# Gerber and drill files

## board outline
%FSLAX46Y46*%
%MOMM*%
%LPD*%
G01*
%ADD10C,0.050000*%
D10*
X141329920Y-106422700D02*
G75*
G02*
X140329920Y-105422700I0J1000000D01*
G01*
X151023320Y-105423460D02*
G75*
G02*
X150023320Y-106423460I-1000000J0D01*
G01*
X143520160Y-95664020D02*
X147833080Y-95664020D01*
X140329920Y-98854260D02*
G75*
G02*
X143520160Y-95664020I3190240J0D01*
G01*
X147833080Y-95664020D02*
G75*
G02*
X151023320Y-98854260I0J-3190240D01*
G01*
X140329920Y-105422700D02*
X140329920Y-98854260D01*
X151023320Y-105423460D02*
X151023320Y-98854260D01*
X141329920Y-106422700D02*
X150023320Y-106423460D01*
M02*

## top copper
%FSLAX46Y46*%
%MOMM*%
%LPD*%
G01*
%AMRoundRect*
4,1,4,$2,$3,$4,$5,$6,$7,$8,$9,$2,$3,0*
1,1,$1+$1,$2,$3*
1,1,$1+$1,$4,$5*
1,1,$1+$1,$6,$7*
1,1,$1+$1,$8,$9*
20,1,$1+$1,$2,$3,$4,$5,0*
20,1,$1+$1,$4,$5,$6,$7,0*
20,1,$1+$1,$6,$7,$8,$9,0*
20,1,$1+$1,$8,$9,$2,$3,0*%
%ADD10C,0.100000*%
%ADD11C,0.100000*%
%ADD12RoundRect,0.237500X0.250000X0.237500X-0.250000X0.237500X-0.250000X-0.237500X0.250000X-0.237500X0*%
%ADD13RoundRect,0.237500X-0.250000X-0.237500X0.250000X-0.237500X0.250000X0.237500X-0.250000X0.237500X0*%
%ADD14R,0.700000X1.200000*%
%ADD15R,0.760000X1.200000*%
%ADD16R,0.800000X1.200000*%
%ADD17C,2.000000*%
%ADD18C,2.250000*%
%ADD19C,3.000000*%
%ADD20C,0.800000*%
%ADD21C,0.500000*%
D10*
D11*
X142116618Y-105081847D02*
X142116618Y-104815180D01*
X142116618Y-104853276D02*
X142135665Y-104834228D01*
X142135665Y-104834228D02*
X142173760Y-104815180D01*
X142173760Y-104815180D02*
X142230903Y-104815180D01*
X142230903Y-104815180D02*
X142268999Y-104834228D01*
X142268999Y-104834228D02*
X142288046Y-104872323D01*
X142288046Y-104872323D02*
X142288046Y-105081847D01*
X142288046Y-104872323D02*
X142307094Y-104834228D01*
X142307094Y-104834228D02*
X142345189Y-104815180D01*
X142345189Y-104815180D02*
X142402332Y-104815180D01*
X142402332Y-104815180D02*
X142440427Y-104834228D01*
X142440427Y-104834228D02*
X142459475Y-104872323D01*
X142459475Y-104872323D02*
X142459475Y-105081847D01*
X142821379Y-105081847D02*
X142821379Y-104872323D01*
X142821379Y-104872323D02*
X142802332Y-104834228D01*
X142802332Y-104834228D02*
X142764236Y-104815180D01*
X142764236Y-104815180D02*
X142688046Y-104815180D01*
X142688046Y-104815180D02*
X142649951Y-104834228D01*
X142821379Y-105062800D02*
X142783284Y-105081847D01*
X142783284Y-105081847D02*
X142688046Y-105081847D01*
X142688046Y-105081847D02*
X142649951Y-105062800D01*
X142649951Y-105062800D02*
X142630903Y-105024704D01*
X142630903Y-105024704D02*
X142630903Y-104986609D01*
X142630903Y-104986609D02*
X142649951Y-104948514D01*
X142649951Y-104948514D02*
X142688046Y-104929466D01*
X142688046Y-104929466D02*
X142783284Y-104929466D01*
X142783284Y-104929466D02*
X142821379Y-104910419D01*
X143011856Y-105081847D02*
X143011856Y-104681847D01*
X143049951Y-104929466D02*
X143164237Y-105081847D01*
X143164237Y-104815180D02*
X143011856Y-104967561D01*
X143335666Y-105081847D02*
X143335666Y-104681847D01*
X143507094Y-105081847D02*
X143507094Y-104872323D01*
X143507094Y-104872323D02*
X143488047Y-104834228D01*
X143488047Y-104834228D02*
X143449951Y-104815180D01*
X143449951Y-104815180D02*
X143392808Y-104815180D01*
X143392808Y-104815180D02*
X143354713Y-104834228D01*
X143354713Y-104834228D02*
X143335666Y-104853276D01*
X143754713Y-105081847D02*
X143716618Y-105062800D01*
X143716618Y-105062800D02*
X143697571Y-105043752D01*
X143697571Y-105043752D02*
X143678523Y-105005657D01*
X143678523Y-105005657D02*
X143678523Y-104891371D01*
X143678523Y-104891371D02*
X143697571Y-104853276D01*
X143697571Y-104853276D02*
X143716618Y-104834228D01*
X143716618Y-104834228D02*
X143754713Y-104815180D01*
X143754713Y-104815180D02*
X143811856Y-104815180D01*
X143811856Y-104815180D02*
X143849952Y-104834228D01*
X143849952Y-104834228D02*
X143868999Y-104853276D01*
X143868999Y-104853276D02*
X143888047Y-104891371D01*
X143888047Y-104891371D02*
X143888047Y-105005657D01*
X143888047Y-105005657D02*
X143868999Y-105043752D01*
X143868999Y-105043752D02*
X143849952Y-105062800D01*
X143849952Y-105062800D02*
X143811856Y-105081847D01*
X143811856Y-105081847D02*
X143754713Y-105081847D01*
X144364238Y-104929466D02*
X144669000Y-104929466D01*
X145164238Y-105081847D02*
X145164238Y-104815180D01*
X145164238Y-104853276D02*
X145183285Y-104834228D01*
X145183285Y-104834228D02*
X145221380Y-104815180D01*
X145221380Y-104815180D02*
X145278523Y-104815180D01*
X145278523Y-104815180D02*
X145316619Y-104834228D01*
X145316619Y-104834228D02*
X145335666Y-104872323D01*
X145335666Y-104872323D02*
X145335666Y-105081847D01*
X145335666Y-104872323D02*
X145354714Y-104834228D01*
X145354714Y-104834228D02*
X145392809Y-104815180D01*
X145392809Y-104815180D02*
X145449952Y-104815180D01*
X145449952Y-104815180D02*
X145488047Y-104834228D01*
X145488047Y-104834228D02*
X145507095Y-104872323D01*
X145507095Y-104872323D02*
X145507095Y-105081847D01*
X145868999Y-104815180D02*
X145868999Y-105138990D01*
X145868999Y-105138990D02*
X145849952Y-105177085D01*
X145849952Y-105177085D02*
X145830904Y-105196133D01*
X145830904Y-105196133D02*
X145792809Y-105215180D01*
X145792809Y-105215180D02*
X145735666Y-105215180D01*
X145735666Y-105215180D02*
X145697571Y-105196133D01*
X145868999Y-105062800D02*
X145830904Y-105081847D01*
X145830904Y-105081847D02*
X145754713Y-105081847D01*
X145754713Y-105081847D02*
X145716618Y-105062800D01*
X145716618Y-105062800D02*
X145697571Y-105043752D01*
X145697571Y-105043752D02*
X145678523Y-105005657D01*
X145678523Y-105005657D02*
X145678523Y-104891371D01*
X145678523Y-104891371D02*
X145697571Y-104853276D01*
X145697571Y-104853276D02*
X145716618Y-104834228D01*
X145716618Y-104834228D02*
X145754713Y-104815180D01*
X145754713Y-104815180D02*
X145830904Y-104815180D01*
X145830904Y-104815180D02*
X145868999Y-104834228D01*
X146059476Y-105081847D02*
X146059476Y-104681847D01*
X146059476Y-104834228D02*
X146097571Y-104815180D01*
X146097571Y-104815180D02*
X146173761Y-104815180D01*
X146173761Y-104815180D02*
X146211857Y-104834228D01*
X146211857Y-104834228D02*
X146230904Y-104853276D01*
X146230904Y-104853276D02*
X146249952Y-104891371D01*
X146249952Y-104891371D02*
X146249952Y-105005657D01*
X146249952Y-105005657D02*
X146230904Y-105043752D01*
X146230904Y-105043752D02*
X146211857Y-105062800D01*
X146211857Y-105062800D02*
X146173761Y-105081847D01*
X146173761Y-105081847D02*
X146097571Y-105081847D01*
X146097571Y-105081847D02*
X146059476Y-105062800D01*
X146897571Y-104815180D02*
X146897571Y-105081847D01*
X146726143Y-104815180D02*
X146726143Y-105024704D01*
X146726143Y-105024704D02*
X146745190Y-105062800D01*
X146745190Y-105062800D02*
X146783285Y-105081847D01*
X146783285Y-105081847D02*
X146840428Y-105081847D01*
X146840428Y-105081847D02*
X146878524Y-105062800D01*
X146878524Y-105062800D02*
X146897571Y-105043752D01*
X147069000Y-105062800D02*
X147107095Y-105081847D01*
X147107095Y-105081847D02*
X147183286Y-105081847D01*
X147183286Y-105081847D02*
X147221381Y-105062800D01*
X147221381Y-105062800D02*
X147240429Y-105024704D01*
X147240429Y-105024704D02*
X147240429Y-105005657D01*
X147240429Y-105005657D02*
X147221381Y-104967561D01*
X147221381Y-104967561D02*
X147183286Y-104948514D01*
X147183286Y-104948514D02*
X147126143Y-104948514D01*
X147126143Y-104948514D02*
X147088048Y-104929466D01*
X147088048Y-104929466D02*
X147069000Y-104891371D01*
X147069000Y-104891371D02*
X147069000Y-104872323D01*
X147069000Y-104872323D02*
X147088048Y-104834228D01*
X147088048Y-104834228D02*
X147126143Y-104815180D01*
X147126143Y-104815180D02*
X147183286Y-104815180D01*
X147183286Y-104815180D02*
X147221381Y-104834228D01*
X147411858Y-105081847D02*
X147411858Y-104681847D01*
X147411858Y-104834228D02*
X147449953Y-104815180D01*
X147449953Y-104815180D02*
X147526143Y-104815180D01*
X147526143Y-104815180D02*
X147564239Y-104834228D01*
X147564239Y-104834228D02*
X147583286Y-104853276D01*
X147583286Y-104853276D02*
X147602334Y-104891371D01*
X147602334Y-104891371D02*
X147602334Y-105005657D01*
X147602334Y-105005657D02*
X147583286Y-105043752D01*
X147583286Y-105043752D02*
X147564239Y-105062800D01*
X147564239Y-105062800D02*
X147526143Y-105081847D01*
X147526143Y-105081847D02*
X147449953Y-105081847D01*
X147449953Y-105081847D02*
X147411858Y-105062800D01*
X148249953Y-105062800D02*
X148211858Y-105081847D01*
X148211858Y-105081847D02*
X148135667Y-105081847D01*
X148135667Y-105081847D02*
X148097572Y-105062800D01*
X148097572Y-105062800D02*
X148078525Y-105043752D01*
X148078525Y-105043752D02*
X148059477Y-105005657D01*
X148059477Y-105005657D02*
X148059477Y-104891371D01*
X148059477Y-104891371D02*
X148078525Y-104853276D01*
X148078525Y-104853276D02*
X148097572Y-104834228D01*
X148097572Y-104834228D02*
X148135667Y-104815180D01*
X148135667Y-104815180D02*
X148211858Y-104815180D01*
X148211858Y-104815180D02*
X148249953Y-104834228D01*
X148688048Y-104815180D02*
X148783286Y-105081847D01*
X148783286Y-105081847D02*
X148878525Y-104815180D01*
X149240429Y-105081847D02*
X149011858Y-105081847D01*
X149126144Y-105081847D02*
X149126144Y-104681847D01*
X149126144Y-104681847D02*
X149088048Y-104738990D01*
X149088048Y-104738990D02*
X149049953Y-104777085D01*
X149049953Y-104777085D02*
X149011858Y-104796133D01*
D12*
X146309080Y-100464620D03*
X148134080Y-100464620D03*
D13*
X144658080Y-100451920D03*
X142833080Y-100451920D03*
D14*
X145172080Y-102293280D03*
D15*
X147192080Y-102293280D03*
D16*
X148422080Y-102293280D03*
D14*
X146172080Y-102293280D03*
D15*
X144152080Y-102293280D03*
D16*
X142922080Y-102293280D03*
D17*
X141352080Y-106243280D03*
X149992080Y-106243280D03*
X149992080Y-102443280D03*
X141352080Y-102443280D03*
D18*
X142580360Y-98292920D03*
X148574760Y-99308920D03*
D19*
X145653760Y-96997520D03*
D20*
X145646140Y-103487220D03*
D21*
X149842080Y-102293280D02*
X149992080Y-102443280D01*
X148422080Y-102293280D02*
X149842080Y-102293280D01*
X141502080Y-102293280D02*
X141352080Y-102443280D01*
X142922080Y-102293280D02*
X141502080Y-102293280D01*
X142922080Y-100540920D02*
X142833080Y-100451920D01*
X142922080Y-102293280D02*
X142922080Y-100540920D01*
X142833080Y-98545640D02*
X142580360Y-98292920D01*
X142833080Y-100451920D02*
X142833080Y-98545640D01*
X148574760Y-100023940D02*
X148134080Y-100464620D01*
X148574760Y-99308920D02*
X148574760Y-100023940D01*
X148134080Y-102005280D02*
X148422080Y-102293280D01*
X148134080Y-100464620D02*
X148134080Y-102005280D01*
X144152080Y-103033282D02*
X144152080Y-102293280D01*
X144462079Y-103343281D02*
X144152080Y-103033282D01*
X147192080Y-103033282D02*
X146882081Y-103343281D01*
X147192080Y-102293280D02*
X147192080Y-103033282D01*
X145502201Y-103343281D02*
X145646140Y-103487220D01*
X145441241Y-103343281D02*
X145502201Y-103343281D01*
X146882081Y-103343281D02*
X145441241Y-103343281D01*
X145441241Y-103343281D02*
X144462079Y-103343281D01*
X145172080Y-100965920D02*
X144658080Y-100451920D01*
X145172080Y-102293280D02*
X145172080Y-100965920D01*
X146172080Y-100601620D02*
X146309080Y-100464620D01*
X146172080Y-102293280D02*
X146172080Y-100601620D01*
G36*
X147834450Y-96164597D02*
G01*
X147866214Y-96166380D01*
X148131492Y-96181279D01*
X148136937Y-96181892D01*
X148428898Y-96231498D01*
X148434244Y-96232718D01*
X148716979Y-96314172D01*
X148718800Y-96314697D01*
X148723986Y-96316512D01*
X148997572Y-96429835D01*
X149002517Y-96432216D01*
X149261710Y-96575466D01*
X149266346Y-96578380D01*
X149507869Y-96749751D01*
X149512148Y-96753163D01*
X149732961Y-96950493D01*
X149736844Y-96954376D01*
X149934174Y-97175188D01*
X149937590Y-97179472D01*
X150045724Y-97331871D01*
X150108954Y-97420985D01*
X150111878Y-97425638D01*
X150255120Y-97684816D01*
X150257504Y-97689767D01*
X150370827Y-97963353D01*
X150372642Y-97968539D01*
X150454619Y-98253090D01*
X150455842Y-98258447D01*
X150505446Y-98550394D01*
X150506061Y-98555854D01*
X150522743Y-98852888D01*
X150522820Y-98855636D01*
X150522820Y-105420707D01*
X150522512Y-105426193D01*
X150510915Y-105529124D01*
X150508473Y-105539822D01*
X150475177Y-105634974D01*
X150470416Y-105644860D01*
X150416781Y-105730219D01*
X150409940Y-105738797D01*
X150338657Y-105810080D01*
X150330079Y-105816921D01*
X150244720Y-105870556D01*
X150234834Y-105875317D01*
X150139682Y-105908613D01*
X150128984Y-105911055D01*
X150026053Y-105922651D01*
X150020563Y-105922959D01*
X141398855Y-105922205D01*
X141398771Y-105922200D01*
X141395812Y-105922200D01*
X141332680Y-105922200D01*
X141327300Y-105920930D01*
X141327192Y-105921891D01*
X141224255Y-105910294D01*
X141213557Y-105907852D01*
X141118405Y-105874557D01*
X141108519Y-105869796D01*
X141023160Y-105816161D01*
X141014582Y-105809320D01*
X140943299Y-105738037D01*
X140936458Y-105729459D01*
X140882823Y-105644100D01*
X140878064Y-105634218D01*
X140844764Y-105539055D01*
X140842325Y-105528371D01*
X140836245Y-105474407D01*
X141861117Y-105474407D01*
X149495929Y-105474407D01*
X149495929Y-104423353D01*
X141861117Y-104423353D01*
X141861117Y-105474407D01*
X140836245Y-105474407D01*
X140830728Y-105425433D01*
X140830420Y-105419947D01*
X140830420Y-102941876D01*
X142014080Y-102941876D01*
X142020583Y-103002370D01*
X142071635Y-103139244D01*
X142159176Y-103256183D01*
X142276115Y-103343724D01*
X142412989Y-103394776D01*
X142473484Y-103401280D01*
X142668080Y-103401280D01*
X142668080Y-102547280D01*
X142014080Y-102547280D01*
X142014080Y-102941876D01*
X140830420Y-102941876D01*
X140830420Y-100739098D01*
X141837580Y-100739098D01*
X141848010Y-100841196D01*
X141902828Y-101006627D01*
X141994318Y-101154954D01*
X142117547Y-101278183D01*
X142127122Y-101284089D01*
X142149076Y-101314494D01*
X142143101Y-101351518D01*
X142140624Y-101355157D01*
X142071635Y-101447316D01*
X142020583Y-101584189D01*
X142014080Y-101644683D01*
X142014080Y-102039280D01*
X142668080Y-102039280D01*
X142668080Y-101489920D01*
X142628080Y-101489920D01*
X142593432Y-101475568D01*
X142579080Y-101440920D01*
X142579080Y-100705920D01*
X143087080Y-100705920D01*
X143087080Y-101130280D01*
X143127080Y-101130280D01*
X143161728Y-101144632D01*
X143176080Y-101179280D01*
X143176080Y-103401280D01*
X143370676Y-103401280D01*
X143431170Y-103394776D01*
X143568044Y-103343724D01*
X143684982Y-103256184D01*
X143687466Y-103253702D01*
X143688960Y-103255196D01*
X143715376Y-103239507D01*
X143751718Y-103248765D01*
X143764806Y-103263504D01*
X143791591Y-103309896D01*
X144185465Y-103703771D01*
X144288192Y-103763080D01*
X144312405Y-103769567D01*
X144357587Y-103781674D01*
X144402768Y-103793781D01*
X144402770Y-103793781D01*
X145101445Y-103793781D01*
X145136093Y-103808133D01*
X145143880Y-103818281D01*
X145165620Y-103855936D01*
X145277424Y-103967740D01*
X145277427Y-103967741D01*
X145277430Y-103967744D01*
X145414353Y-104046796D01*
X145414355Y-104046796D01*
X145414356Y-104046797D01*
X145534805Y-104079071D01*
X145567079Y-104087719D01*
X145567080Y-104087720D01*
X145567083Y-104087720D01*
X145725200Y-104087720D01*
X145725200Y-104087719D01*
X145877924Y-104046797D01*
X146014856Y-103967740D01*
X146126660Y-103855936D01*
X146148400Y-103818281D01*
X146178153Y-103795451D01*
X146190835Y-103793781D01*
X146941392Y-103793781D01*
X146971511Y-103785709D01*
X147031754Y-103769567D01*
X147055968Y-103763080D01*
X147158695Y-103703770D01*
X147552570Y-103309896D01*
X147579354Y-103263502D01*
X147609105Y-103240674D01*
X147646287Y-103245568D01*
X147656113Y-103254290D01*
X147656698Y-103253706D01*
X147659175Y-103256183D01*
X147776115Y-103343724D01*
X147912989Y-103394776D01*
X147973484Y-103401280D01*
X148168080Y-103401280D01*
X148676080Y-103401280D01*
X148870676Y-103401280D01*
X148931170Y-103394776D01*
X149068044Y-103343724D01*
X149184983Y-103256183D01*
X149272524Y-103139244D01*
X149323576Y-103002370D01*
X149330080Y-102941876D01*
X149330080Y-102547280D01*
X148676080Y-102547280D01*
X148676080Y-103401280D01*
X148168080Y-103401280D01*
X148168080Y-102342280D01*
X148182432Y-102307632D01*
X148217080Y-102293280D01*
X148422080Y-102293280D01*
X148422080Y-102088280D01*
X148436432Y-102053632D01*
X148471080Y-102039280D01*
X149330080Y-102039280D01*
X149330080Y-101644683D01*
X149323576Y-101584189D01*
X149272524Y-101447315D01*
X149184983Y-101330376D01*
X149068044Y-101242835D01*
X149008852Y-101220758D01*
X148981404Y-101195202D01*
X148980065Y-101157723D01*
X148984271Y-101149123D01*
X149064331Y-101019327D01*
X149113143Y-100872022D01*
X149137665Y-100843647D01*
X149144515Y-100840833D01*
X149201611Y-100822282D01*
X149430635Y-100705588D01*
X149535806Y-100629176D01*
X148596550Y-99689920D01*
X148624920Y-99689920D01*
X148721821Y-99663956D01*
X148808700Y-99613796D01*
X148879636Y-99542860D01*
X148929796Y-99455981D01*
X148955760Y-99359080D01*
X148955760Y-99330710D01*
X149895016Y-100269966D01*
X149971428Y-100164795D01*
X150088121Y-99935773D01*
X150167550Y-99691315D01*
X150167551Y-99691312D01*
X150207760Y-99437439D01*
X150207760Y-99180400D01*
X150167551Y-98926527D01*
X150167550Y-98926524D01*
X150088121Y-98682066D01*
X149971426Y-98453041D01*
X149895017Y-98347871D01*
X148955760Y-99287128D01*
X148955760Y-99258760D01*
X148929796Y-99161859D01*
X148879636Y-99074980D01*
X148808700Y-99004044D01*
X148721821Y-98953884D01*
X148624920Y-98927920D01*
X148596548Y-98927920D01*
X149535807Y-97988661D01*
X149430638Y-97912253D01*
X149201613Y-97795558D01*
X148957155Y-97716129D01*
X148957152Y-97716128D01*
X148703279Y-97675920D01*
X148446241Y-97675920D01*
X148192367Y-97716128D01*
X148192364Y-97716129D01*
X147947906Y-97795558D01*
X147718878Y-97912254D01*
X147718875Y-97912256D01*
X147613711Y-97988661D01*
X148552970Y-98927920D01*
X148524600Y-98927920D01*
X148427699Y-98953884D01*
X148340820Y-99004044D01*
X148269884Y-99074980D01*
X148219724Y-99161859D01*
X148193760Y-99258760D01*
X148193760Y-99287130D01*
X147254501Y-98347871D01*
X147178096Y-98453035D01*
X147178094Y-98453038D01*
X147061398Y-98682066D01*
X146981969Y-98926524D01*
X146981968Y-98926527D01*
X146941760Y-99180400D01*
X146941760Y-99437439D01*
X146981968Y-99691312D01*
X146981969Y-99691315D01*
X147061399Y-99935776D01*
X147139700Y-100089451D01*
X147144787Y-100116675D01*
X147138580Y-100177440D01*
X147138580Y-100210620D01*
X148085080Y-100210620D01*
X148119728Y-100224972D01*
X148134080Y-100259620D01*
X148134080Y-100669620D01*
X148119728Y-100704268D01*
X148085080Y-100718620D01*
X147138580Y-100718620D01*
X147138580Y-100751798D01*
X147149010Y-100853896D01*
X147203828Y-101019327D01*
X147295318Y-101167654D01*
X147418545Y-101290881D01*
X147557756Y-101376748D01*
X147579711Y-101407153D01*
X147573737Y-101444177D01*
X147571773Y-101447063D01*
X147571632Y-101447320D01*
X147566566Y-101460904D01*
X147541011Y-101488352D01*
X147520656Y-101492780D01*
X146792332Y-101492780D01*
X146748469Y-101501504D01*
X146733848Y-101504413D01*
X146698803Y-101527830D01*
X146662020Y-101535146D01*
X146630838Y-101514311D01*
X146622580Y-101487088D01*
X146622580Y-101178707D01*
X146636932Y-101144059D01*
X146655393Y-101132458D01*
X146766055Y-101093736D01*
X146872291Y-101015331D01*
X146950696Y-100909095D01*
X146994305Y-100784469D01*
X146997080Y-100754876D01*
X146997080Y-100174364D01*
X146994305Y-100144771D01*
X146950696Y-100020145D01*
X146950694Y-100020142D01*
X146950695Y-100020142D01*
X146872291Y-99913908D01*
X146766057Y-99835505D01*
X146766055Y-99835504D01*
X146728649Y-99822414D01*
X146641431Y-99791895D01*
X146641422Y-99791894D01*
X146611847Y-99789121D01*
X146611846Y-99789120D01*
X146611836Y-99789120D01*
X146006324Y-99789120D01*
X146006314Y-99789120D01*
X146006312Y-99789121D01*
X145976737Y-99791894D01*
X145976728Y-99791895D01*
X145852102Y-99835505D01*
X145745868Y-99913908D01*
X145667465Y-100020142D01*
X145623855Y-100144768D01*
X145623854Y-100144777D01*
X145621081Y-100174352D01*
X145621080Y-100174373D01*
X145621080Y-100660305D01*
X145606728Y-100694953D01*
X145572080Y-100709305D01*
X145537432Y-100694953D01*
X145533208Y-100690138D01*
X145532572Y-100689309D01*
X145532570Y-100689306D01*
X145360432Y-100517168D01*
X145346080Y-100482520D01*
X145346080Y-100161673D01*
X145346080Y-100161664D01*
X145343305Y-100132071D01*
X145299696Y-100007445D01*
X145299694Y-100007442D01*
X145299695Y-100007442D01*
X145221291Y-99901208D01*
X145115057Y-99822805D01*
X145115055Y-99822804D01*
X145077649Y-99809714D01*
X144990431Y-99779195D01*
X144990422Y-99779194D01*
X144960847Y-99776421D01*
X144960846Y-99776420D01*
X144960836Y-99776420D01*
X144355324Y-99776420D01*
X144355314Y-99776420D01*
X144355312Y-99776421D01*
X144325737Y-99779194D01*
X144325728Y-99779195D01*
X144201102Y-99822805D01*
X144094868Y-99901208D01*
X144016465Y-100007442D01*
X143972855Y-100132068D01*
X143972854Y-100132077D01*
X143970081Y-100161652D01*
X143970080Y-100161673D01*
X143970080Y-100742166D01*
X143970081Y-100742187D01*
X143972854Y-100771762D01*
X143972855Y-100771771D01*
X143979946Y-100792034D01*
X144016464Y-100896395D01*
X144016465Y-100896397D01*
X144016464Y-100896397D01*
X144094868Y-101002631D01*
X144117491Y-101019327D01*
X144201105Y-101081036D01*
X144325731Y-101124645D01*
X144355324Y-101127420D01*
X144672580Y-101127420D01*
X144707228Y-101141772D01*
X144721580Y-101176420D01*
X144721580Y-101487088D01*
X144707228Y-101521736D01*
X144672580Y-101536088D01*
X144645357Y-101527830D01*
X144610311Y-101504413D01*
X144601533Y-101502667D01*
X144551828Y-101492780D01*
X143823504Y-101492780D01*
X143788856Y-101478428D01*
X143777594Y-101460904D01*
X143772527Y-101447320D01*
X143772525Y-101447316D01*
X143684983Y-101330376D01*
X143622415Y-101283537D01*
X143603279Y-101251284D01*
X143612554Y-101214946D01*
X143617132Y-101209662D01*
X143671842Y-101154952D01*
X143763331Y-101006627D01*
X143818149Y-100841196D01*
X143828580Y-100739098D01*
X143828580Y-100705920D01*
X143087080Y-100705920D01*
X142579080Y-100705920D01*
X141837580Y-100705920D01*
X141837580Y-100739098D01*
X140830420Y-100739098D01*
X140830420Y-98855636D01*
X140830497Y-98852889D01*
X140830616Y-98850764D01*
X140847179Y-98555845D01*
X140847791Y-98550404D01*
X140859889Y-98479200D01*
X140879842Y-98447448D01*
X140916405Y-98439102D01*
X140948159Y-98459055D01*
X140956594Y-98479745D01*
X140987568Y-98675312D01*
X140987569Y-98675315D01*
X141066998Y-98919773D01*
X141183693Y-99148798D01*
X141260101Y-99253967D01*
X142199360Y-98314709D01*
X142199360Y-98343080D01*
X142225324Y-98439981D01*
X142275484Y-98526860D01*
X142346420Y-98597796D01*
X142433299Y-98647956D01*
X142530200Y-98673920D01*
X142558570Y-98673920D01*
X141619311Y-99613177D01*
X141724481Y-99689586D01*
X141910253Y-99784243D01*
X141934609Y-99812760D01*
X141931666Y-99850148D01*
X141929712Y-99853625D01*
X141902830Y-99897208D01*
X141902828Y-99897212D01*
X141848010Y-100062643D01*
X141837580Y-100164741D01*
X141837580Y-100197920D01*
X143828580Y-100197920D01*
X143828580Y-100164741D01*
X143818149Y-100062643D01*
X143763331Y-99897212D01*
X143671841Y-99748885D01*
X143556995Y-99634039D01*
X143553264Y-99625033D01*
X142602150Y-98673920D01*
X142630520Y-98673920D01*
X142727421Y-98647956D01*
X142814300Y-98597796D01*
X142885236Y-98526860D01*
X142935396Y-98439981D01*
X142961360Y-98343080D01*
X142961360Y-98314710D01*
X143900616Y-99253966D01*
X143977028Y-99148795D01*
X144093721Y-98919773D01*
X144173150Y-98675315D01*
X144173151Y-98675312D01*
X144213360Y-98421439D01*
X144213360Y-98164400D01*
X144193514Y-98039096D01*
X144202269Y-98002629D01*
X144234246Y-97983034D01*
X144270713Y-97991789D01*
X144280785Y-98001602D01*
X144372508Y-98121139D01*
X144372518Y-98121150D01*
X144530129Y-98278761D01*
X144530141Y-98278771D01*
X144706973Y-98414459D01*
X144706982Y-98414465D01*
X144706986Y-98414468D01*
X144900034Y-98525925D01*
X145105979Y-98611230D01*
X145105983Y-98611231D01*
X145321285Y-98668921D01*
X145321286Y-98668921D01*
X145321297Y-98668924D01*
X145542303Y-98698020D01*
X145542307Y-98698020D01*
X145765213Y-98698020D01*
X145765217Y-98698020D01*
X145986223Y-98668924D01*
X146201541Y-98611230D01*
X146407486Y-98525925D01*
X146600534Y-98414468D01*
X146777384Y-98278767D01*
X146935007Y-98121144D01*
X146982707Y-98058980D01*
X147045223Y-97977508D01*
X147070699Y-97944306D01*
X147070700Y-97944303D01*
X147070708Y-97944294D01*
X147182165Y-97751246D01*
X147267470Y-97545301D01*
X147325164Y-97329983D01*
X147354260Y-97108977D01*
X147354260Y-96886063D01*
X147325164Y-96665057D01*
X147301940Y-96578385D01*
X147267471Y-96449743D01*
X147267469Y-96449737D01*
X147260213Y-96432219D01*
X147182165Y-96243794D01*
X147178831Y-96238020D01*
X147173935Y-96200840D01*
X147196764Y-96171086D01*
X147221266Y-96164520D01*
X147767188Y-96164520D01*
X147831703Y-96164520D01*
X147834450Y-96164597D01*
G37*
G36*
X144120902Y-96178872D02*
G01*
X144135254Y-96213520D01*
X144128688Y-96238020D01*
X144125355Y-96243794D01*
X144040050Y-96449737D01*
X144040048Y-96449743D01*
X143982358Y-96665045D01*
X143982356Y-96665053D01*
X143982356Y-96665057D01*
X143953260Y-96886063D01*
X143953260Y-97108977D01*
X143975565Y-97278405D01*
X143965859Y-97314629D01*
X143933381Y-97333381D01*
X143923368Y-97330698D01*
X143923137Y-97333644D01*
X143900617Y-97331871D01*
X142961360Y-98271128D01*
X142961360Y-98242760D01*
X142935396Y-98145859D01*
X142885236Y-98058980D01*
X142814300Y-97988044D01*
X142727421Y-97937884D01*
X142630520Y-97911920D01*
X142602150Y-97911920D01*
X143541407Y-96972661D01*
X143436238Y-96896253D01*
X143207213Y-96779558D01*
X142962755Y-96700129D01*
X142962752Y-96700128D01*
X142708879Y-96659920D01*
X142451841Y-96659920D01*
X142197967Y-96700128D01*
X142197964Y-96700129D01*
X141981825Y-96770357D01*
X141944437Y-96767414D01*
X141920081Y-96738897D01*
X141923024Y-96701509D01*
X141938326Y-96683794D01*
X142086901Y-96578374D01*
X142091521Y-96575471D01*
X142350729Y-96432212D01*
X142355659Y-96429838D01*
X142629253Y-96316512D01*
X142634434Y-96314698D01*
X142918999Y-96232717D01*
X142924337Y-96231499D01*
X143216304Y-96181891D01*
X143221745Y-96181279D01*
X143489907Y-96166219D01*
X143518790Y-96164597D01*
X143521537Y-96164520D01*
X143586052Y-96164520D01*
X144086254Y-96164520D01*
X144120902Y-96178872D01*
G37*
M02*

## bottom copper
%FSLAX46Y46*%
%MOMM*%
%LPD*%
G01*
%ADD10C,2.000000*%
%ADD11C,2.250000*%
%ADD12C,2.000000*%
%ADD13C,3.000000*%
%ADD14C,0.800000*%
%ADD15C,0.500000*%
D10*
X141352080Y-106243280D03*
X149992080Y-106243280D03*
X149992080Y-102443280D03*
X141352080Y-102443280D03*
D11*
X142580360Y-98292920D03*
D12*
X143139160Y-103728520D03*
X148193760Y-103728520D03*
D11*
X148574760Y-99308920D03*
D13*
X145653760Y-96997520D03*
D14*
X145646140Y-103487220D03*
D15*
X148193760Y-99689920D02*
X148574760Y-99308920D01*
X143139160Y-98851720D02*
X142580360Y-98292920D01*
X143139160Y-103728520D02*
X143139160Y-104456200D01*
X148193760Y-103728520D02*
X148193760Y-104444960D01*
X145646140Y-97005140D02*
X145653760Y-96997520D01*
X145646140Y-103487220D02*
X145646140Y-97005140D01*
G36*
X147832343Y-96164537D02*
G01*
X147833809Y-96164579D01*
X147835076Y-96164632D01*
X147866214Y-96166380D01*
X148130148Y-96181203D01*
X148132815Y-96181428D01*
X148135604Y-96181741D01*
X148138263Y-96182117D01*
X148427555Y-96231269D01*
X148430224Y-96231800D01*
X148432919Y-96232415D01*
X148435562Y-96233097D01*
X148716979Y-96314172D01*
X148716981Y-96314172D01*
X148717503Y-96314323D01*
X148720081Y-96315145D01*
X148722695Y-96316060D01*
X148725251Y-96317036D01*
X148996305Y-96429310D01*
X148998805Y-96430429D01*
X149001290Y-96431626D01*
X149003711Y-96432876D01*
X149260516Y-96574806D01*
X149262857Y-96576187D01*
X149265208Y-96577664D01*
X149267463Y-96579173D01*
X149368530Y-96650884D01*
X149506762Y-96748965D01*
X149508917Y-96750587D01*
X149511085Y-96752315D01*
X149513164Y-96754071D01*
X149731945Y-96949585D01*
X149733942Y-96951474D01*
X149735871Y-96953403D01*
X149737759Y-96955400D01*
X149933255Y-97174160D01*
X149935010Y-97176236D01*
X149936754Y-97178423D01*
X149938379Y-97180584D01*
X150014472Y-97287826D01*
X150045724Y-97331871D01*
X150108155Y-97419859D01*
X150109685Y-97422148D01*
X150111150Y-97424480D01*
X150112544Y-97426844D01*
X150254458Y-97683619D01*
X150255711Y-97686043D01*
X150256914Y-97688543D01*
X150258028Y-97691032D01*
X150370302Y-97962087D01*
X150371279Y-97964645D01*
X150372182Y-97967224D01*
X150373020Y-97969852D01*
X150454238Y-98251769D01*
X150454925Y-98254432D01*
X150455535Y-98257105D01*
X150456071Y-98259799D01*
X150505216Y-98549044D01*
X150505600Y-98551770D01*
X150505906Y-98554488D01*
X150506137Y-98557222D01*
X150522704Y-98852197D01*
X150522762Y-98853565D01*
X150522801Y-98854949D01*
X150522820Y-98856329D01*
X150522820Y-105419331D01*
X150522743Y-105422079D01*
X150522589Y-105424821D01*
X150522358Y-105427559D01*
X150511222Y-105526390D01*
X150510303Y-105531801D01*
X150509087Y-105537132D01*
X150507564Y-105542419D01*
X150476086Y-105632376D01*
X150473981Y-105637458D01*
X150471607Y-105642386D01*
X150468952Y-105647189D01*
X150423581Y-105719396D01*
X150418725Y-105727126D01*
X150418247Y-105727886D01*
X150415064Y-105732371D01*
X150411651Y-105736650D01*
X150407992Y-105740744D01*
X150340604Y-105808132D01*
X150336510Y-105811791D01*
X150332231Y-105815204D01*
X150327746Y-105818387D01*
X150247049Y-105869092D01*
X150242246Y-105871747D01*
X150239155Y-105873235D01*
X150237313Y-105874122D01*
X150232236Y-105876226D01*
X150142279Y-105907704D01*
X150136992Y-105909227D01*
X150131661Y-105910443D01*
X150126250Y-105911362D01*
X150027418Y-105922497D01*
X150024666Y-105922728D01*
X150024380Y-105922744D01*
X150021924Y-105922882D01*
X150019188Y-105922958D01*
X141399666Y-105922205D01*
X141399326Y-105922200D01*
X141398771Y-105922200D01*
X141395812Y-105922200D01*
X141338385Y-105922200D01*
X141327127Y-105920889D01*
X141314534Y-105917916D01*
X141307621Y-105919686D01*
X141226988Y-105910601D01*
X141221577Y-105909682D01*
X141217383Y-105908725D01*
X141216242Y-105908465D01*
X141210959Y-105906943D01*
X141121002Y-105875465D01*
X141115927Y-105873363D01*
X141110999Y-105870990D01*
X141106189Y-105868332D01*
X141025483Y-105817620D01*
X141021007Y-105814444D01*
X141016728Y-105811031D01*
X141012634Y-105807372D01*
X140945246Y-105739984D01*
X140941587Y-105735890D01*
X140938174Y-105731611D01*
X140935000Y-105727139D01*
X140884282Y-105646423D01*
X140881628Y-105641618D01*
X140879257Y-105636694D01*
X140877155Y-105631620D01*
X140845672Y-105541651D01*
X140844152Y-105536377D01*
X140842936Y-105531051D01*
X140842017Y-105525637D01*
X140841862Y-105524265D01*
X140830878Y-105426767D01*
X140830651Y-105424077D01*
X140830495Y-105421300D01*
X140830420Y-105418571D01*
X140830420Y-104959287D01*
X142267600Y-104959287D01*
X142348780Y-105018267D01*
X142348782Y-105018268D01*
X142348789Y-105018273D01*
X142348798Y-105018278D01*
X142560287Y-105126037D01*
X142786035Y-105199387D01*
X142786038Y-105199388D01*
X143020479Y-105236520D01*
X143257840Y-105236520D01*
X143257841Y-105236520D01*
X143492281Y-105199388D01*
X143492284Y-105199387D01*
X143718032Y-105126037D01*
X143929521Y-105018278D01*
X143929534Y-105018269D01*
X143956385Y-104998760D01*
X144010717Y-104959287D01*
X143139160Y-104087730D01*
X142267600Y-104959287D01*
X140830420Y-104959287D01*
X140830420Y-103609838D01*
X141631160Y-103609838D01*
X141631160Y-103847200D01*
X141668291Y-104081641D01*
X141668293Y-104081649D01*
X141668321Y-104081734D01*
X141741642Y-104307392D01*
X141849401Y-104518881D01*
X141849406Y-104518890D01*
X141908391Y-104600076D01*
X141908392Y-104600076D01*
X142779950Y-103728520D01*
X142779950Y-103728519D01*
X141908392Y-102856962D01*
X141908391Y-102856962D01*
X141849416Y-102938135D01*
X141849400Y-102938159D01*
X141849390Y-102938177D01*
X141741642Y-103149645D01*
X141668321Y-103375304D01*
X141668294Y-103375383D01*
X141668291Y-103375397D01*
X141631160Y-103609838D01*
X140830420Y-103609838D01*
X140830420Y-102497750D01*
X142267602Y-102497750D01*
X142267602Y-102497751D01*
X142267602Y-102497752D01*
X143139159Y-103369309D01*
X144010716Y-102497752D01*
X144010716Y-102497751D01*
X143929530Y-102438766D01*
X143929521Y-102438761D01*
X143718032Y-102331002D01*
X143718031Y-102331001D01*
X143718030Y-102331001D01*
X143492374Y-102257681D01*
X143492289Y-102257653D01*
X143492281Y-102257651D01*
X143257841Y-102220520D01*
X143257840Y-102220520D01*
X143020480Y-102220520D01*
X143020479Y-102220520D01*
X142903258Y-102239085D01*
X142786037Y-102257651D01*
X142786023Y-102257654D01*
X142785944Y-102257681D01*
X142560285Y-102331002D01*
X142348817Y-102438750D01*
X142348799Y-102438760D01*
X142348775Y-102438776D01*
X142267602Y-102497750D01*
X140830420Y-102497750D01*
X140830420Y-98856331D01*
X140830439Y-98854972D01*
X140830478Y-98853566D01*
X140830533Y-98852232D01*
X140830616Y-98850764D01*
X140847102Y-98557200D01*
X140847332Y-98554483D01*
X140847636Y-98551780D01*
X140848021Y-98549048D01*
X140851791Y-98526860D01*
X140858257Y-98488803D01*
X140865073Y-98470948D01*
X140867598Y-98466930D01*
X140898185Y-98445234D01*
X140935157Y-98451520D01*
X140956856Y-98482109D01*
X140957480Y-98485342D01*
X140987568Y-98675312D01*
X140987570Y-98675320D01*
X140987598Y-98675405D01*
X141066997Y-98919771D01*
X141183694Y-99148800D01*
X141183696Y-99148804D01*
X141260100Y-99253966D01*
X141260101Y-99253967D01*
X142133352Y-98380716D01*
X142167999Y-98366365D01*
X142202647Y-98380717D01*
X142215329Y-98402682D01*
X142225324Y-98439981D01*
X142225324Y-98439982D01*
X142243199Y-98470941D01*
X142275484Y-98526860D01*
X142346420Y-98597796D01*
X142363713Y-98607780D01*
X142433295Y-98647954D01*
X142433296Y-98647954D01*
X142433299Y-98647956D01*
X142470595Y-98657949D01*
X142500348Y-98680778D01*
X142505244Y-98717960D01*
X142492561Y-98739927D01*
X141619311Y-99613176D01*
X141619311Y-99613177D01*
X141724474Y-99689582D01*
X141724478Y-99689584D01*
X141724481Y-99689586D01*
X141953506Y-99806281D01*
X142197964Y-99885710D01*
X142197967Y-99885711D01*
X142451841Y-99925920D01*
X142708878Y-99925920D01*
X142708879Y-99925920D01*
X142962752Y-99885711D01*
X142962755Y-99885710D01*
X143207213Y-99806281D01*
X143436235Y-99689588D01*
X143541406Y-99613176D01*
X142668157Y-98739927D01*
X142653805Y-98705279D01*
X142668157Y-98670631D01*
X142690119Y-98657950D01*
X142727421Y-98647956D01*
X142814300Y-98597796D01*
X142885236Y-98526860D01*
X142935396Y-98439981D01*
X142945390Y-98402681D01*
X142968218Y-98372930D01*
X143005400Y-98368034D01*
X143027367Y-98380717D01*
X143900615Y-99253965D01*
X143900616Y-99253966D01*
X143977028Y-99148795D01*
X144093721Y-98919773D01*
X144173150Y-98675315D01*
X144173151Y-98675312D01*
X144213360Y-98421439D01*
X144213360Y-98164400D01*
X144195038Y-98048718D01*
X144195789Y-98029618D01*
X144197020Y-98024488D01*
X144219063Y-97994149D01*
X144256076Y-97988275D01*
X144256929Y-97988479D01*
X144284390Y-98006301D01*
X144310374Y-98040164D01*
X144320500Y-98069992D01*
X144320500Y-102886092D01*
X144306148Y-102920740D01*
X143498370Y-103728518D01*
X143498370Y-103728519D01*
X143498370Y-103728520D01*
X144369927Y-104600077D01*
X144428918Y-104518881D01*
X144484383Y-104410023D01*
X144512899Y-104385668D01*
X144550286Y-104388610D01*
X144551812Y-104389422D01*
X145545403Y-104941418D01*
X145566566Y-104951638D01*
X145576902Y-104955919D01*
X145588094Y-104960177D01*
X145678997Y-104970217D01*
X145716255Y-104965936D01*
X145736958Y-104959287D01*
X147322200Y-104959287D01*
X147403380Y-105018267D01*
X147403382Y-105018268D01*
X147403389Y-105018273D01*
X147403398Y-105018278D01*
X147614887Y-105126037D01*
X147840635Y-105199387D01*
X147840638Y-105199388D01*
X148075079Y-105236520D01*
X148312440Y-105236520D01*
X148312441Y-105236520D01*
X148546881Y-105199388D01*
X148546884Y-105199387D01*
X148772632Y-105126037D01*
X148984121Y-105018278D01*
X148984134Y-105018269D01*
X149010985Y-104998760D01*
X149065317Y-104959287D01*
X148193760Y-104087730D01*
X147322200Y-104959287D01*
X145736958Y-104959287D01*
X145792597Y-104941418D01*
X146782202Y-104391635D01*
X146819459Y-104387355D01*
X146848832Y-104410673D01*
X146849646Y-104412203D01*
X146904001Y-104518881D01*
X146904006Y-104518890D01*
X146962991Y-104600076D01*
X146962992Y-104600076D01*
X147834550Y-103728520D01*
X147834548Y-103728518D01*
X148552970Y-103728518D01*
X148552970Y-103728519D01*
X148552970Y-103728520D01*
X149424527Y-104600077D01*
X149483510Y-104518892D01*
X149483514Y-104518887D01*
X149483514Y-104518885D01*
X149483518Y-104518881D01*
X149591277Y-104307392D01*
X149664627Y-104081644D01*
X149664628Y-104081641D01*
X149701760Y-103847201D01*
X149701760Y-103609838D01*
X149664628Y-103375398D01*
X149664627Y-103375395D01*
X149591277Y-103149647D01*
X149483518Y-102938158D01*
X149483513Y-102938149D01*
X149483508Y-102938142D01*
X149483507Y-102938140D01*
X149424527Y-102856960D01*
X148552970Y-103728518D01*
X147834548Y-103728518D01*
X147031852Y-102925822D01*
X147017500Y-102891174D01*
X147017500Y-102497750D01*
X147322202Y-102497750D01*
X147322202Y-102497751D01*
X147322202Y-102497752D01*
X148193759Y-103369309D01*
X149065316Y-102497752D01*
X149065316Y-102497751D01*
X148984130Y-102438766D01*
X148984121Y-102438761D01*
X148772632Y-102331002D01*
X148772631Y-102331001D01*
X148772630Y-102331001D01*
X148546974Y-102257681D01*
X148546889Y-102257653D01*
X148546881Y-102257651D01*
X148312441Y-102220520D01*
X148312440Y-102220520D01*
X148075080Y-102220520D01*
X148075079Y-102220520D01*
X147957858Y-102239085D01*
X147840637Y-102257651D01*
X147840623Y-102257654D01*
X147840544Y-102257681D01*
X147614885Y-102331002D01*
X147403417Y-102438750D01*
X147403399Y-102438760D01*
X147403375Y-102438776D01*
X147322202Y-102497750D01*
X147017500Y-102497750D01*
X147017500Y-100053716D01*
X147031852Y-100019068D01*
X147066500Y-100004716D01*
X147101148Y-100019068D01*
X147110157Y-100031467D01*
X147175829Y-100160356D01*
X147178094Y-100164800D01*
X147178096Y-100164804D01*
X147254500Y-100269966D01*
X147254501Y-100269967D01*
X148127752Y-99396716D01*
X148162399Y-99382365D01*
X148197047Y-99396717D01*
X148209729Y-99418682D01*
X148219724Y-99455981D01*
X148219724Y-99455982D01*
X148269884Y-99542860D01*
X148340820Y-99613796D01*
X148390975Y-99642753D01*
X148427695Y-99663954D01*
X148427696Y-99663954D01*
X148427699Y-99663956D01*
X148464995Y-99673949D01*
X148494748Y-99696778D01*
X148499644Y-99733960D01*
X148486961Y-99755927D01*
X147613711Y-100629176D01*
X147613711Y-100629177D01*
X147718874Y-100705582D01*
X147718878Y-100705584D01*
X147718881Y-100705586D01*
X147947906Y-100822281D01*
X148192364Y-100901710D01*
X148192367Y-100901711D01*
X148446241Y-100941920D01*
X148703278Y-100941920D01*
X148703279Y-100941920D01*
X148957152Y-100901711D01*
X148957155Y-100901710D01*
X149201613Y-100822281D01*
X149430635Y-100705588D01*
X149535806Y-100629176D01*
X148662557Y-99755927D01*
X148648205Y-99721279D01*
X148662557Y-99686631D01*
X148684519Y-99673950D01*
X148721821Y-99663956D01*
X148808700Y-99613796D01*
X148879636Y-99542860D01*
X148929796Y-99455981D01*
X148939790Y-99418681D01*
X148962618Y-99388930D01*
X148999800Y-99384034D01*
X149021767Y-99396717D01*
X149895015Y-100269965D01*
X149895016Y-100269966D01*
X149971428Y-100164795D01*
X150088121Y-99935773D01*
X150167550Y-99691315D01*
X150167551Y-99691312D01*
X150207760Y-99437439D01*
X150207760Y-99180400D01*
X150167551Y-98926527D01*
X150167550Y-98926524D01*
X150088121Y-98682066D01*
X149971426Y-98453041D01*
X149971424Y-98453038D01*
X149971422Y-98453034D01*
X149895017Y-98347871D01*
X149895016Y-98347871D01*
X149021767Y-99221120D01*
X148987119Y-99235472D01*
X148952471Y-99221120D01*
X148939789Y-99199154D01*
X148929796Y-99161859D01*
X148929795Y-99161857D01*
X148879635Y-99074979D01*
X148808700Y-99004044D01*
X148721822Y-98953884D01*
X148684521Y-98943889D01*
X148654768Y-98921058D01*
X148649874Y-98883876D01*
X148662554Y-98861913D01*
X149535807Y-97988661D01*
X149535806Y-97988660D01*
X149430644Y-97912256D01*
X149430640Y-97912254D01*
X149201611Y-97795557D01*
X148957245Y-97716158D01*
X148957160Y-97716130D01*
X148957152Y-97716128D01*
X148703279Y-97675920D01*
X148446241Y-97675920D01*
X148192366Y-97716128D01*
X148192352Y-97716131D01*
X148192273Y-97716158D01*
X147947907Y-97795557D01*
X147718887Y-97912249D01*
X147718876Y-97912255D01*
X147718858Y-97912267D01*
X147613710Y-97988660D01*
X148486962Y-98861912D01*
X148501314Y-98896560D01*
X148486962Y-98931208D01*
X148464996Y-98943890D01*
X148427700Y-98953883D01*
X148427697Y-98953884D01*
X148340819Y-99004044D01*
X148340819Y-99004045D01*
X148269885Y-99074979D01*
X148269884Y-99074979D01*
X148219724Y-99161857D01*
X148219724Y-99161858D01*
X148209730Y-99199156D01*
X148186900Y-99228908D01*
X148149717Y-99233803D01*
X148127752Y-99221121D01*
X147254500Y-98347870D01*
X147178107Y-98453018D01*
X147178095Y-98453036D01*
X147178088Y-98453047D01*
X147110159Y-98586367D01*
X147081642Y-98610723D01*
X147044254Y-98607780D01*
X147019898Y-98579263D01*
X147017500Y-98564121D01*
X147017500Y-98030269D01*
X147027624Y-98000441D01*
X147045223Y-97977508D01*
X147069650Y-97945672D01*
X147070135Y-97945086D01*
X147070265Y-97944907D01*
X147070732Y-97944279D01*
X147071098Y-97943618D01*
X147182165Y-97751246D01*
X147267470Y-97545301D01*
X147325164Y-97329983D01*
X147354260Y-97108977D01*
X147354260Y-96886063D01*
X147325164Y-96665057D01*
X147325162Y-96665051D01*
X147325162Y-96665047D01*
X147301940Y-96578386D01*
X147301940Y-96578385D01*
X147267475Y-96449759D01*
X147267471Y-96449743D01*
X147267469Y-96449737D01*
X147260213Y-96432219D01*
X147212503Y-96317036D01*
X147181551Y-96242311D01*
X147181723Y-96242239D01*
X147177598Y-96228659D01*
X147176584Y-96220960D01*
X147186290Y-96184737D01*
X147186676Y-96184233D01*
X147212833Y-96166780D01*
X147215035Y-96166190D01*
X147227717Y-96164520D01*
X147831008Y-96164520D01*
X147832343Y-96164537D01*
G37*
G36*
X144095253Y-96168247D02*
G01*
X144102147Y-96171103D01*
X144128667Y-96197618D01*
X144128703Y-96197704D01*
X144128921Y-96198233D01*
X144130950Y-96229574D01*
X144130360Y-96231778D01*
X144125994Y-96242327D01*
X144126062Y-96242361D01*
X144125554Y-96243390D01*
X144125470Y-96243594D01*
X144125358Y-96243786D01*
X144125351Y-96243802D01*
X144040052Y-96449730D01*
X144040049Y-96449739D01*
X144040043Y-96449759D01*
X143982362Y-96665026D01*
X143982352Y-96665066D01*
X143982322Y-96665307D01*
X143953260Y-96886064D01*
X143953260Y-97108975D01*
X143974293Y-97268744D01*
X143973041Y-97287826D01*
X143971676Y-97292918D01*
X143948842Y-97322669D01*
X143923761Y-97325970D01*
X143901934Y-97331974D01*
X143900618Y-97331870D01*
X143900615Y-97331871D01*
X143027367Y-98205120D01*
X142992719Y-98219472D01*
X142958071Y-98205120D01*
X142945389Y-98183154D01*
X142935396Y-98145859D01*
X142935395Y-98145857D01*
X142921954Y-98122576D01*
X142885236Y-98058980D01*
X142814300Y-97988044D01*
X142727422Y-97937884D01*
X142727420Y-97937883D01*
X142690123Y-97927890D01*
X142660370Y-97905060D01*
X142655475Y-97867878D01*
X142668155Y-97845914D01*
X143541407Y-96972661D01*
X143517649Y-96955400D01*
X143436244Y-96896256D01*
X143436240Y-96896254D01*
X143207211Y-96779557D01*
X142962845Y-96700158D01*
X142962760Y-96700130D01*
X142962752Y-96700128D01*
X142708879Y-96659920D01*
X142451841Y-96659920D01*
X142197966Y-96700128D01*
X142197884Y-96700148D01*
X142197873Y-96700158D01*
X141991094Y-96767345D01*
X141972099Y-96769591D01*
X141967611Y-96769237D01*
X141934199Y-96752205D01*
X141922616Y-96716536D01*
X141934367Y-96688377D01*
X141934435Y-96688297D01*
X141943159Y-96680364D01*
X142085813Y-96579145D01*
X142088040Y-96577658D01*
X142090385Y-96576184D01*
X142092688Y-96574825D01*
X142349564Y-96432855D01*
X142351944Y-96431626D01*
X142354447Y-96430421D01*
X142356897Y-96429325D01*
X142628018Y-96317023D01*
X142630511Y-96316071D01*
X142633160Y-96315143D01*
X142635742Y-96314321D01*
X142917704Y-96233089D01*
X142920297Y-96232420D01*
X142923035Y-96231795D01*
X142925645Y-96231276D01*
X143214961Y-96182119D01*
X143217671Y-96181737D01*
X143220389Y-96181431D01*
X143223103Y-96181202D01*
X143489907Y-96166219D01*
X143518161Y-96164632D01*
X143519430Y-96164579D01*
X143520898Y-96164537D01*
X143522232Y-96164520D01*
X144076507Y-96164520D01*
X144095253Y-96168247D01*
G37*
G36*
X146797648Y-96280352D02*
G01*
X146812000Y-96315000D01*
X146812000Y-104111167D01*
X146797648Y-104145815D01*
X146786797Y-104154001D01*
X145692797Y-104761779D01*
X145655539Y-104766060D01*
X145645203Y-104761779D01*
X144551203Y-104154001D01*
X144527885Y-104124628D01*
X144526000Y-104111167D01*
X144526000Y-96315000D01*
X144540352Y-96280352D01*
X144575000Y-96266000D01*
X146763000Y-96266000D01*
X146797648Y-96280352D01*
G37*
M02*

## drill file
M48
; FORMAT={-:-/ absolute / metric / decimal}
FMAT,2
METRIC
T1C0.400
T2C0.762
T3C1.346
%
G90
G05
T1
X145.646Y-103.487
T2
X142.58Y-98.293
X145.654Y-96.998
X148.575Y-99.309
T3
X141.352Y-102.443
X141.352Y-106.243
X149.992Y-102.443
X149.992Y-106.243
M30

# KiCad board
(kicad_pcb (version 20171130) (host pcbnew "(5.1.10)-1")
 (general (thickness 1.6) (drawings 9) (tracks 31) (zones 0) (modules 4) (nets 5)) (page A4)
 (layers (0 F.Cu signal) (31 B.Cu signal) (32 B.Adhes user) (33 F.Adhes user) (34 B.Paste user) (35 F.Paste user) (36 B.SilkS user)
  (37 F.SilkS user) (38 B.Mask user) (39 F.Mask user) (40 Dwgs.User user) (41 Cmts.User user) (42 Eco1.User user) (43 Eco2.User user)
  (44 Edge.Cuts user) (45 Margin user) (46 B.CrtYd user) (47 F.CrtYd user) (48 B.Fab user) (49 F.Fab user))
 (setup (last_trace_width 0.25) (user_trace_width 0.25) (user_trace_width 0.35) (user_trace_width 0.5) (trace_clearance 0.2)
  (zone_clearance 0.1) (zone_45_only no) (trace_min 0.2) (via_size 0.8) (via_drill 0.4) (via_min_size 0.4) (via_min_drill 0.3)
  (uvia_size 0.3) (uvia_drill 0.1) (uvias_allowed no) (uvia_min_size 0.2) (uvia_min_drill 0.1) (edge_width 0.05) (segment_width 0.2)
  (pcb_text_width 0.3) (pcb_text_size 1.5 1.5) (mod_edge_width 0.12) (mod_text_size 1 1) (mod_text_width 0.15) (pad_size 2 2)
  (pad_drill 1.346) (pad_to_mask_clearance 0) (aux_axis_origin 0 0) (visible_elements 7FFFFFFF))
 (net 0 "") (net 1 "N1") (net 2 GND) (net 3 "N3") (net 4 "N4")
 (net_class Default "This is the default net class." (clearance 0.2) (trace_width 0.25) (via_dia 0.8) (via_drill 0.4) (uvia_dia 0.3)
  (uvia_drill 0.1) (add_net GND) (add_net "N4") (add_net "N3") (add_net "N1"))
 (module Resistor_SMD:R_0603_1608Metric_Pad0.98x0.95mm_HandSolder (layer F.Cu) (at 147.22158 100.46462 180)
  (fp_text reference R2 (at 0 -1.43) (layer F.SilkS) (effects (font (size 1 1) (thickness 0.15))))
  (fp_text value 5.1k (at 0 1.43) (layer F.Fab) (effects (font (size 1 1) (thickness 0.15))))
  (pad 2 smd roundrect (at 0.9125 0 180) (size 0.975 0.95) (layers F.Cu F.Paste F.Mask) (roundrect_rratio 0.25) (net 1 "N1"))
  (pad 1 smd roundrect (at -0.9125 0 180) (size 0.975 0.95) (layers F.Cu F.Paste F.Mask) (roundrect_rratio 0.25) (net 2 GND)))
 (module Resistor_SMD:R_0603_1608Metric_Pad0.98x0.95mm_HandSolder (layer F.Cu) (at 143.74558 100.45192)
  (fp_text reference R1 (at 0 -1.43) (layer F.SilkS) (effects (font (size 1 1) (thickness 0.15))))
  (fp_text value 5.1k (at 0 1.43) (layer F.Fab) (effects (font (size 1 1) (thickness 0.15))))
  (pad 2 smd roundrect (at 0.9125 0) (size 0.975 0.95) (layers F.Cu F.Paste F.Mask) (roundrect_rratio 0.25) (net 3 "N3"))
  (pad 1 smd roundrect (at -0.9125 0) (size 0.975 0.95) (layers F.Cu F.Paste F.Mask) (roundrect_rratio 0.25) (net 2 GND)))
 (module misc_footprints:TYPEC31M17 (layer F.Cu) (at 145.67208 104.79328)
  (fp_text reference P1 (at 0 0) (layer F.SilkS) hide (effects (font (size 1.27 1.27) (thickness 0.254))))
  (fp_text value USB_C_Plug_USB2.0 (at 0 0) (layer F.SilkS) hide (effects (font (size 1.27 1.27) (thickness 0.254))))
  (pad A5 smd rect (at -0.5 -2.5) (size 0.7 1.2) (layers F.Cu F.Paste F.Mask) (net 3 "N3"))
  (pad A9 smd rect (at 1.52 -2.5) (size 0.76 1.2) (layers F.Cu F.Paste F.Mask) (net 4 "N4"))
  (pad A12 smd rect (at 2.75 -2.5) (size 0.8 1.2) (layers F.Cu F.Paste F.Mask) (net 2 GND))
  (pad B5 smd rect (at 0.5 -2.5) (size 0.7 1.2) (layers F.Cu F.Paste F.Mask) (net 1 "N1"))
  (pad B9 smd rect (at -1.52 -2.5) (size 0.76 1.2) (layers F.Cu F.Paste F.Mask) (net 4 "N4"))
  (pad B12 smd rect (at -2.75 -2.5) (size 0.8 1.2) (layers F.Cu F.Paste F.Mask) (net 2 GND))
  (pad MH1 thru_hole circle (at -4.32 1.45) (size 2 2) (drill 1.346) (layers *.Cu *.Mask) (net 2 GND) (zone_connect 2))
  (pad MH2 thru_hole circle (at 4.32 1.45) (size 2 2) (drill 1.346) (layers *.Cu *.Mask) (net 2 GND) (zone_connect 2))
  (pad MH3 thru_hole circle (at 4.32 -2.35) (size 2 2) (drill 1.346) (layers *.Cu *.Mask) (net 2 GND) (zone_connect 2))
  (pad MH4 thru_hole circle (at -4.32 -2.35) (size 2 2) (drill 1.346) (layers *.Cu *.Mask) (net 2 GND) (zone_connect 2)))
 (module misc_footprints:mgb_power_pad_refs (layer F.Cu) (at 150.12416 101.29012)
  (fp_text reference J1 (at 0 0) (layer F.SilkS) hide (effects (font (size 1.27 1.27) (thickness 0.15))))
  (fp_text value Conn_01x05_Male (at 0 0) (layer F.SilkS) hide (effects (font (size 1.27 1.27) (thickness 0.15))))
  (pad 2 thru_hole circle (at -7.5438 -2.9972) (size 2.25 2.25) (drill 0.762) (layers *.Cu *.Mask) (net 2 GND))
  (pad 4 smd circle (at -6.985 2.4384) (size 2 2) (layers B.Cu B.Paste B.Mask) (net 2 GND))
  (pad 5 smd circle (at -1.9304 2.4384) (size 2 2) (layers B.Cu B.Paste B.Mask) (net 2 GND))
  (pad 3 thru_hole circle (at -1.5494 -1.9812) (size 2.25 2.25) (drill 0.762) (layers *.Cu *.Mask) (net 2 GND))
  (pad 1 thru_hole circle (at -4.4704 -4.2926) (size 3 3) (drill 0.762) (layers *.Cu *.Mask) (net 4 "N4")))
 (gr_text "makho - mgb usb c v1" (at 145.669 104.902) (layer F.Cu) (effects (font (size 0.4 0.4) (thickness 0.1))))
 (gr_arc (start 141.32992 105.4227) (end 140.32992 105.4227) (angle -90) (layer Edge.Cuts) (width 0.05))
 (gr_arc (start 150.02332 105.42346) (end 150.02332 106.42346) (angle -90) (layer Edge.Cuts) (width 0.05))
 (gr_line (start 143.52016 95.66402) (end 147.83308 95.66402) (layer Edge.Cuts) (width 0.05))
 (gr_arc (start 143.52016 98.85426) (end 143.52016 95.66402) (angle -90) (layer Edge.Cuts) (width 0.05))
 (gr_arc (start 147.83308 98.85426) (end 151.02332 98.85426) (angle -90) (layer Edge.Cuts) (width 0.05))
 (gr_line (start 140.32992 105.4227) (end 140.32992 98.85426) (layer Edge.Cuts) (width 0.05))
 (gr_line (start 151.02332 105.42346) (end 151.02332 98.85426) (layer Edge.Cuts) (width 0.05))
 (gr_line (start 141.32992 106.4227) (end 150.02332 106.42346) (layer Edge.Cuts) (width 0.05))
 (segment (start 149.84208 102.29328) (end 149.99208 102.44328) (width 0.5) (layer F.Cu) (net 2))
 (segment (start 148.42208 102.29328) (end 149.84208 102.29328) (width 0.5) (layer F.Cu) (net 2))
 (segment (start 141.50208 102.29328) (end 141.35208 102.44328) (width 0.5) (layer F.Cu) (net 2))
 (segment (start 142.92208 102.29328) (end 141.50208 102.29328) (width 0.5) (layer F.Cu) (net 2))
 (segment (start 142.92208 100.54092) (end 142.83308 100.45192) (width 0.5) (layer F.Cu) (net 2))
 (segment (start 142.92208 102.29328) (end 142.92208 100.54092) (width 0.5) (layer F.Cu) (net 2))
 (segment (start 142.83308 98.54564) (end 142.58036 98.29292) (width 0.5) (layer F.Cu) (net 2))
 (segment (start 142.83308 100.45192) (end 142.83308 98.54564) (width 0.5) (layer F.Cu) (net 2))
 (segment (start 148.57476 100.02394) (end 148.13408 100.46462) (width 0.5) (layer F.Cu) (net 2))
 (segment (start 148.57476 99.30892) (end 148.57476 100.02394) (width 0.5) (layer F.Cu) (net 2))
 (segment (start 148.13408 102.00528) (end 148.42208 102.29328) (width 0.5) (layer F.Cu) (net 2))
 (segment (start 148.13408 100.46462) (end 148.13408 102.00528) (width 0.5) (layer F.Cu) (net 2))
 (segment (start 148.19376 99.68992) (end 148.57476 99.30892) (width 0.5) (layer B.Cu) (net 2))
 (segment (start 143.13916 98.85172) (end 142.58036 98.29292) (width 0.5) (layer B.Cu) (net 2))
 (segment (start 143.13916 103.72852) (end 143.13916 104.4562) (width 0.5) (layer B.Cu) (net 2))
 (segment (start 148.19376 103.72852) (end 148.19376 104.44496) (width 0.5) (layer B.Cu) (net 2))
 (segment (start 144.15208 103.033282) (end 144.15208 102.29328) (width 0.5) (layer F.Cu) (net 4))
 (segment (start 144.462079 103.343281) (end 144.15208 103.033282) (width 0.5) (layer F.Cu) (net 4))
 (segment (start 147.19208 103.033282) (end 146.882081 103.343281) (width 0.5) (layer F.Cu) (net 4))
 (segment (start 147.19208 102.29328) (end 147.19208 103.033282) (width 0.5) (layer F.Cu) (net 4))
 (segment (start 145.502201 103.343281) (end 145.64614 103.48722) (width 0.5) (layer F.Cu) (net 4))
 (segment (start 145.441241 103.343281) (end 145.502201 103.343281) (width 0.5) (layer F.Cu) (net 4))
 (via (at 145.64614 103.48722) (size 0.8) (drill 0.4) (layers F.Cu B.Cu) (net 4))
 (segment (start 146.882081 103.343281) (end 145.441241 103.343281) (width 0.5) (layer F.Cu) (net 4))
 (segment (start 145.441241 103.343281) (end 144.462079 103.343281) (width 0.5) (layer F.Cu) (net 4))
 (segment (start 145.64614 97.00514) (end 145.65376 96.99752) (width 0.5) (layer B.Cu) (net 4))
 (segment (start 145.64614 103.48722) (end 145.64614 97.00514) (width 0.5) (layer B.Cu) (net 4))
 (segment (start 145.17208 100.96592) (end 144.65808 100.45192) (width 0.5) (layer F.Cu) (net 3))
 (segment (start 145.17208 102.29328) (end 145.17208 100.96592) (width 0.5) (layer F.Cu) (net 3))
 (segment (start 146.17208 100.60162) (end 146.30908 100.46462) (width 0.5) (layer F.Cu) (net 1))
 (segment (start 146.17208 102.29328) (end 146.17208 100.60162) (width 0.5) (layer F.Cu) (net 1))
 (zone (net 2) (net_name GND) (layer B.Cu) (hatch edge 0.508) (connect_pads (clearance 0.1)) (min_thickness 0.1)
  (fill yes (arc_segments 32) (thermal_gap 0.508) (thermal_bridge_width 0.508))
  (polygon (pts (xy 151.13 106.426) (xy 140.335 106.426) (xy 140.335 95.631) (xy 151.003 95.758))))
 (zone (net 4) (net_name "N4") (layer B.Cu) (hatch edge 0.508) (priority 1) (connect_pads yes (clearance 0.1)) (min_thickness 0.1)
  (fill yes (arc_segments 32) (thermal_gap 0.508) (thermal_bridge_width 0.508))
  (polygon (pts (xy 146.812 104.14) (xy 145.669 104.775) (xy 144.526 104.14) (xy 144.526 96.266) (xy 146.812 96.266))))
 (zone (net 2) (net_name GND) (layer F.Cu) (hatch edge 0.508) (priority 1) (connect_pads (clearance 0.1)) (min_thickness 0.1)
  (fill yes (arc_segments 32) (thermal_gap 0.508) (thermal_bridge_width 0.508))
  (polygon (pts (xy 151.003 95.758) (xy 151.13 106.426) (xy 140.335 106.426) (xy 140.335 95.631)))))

